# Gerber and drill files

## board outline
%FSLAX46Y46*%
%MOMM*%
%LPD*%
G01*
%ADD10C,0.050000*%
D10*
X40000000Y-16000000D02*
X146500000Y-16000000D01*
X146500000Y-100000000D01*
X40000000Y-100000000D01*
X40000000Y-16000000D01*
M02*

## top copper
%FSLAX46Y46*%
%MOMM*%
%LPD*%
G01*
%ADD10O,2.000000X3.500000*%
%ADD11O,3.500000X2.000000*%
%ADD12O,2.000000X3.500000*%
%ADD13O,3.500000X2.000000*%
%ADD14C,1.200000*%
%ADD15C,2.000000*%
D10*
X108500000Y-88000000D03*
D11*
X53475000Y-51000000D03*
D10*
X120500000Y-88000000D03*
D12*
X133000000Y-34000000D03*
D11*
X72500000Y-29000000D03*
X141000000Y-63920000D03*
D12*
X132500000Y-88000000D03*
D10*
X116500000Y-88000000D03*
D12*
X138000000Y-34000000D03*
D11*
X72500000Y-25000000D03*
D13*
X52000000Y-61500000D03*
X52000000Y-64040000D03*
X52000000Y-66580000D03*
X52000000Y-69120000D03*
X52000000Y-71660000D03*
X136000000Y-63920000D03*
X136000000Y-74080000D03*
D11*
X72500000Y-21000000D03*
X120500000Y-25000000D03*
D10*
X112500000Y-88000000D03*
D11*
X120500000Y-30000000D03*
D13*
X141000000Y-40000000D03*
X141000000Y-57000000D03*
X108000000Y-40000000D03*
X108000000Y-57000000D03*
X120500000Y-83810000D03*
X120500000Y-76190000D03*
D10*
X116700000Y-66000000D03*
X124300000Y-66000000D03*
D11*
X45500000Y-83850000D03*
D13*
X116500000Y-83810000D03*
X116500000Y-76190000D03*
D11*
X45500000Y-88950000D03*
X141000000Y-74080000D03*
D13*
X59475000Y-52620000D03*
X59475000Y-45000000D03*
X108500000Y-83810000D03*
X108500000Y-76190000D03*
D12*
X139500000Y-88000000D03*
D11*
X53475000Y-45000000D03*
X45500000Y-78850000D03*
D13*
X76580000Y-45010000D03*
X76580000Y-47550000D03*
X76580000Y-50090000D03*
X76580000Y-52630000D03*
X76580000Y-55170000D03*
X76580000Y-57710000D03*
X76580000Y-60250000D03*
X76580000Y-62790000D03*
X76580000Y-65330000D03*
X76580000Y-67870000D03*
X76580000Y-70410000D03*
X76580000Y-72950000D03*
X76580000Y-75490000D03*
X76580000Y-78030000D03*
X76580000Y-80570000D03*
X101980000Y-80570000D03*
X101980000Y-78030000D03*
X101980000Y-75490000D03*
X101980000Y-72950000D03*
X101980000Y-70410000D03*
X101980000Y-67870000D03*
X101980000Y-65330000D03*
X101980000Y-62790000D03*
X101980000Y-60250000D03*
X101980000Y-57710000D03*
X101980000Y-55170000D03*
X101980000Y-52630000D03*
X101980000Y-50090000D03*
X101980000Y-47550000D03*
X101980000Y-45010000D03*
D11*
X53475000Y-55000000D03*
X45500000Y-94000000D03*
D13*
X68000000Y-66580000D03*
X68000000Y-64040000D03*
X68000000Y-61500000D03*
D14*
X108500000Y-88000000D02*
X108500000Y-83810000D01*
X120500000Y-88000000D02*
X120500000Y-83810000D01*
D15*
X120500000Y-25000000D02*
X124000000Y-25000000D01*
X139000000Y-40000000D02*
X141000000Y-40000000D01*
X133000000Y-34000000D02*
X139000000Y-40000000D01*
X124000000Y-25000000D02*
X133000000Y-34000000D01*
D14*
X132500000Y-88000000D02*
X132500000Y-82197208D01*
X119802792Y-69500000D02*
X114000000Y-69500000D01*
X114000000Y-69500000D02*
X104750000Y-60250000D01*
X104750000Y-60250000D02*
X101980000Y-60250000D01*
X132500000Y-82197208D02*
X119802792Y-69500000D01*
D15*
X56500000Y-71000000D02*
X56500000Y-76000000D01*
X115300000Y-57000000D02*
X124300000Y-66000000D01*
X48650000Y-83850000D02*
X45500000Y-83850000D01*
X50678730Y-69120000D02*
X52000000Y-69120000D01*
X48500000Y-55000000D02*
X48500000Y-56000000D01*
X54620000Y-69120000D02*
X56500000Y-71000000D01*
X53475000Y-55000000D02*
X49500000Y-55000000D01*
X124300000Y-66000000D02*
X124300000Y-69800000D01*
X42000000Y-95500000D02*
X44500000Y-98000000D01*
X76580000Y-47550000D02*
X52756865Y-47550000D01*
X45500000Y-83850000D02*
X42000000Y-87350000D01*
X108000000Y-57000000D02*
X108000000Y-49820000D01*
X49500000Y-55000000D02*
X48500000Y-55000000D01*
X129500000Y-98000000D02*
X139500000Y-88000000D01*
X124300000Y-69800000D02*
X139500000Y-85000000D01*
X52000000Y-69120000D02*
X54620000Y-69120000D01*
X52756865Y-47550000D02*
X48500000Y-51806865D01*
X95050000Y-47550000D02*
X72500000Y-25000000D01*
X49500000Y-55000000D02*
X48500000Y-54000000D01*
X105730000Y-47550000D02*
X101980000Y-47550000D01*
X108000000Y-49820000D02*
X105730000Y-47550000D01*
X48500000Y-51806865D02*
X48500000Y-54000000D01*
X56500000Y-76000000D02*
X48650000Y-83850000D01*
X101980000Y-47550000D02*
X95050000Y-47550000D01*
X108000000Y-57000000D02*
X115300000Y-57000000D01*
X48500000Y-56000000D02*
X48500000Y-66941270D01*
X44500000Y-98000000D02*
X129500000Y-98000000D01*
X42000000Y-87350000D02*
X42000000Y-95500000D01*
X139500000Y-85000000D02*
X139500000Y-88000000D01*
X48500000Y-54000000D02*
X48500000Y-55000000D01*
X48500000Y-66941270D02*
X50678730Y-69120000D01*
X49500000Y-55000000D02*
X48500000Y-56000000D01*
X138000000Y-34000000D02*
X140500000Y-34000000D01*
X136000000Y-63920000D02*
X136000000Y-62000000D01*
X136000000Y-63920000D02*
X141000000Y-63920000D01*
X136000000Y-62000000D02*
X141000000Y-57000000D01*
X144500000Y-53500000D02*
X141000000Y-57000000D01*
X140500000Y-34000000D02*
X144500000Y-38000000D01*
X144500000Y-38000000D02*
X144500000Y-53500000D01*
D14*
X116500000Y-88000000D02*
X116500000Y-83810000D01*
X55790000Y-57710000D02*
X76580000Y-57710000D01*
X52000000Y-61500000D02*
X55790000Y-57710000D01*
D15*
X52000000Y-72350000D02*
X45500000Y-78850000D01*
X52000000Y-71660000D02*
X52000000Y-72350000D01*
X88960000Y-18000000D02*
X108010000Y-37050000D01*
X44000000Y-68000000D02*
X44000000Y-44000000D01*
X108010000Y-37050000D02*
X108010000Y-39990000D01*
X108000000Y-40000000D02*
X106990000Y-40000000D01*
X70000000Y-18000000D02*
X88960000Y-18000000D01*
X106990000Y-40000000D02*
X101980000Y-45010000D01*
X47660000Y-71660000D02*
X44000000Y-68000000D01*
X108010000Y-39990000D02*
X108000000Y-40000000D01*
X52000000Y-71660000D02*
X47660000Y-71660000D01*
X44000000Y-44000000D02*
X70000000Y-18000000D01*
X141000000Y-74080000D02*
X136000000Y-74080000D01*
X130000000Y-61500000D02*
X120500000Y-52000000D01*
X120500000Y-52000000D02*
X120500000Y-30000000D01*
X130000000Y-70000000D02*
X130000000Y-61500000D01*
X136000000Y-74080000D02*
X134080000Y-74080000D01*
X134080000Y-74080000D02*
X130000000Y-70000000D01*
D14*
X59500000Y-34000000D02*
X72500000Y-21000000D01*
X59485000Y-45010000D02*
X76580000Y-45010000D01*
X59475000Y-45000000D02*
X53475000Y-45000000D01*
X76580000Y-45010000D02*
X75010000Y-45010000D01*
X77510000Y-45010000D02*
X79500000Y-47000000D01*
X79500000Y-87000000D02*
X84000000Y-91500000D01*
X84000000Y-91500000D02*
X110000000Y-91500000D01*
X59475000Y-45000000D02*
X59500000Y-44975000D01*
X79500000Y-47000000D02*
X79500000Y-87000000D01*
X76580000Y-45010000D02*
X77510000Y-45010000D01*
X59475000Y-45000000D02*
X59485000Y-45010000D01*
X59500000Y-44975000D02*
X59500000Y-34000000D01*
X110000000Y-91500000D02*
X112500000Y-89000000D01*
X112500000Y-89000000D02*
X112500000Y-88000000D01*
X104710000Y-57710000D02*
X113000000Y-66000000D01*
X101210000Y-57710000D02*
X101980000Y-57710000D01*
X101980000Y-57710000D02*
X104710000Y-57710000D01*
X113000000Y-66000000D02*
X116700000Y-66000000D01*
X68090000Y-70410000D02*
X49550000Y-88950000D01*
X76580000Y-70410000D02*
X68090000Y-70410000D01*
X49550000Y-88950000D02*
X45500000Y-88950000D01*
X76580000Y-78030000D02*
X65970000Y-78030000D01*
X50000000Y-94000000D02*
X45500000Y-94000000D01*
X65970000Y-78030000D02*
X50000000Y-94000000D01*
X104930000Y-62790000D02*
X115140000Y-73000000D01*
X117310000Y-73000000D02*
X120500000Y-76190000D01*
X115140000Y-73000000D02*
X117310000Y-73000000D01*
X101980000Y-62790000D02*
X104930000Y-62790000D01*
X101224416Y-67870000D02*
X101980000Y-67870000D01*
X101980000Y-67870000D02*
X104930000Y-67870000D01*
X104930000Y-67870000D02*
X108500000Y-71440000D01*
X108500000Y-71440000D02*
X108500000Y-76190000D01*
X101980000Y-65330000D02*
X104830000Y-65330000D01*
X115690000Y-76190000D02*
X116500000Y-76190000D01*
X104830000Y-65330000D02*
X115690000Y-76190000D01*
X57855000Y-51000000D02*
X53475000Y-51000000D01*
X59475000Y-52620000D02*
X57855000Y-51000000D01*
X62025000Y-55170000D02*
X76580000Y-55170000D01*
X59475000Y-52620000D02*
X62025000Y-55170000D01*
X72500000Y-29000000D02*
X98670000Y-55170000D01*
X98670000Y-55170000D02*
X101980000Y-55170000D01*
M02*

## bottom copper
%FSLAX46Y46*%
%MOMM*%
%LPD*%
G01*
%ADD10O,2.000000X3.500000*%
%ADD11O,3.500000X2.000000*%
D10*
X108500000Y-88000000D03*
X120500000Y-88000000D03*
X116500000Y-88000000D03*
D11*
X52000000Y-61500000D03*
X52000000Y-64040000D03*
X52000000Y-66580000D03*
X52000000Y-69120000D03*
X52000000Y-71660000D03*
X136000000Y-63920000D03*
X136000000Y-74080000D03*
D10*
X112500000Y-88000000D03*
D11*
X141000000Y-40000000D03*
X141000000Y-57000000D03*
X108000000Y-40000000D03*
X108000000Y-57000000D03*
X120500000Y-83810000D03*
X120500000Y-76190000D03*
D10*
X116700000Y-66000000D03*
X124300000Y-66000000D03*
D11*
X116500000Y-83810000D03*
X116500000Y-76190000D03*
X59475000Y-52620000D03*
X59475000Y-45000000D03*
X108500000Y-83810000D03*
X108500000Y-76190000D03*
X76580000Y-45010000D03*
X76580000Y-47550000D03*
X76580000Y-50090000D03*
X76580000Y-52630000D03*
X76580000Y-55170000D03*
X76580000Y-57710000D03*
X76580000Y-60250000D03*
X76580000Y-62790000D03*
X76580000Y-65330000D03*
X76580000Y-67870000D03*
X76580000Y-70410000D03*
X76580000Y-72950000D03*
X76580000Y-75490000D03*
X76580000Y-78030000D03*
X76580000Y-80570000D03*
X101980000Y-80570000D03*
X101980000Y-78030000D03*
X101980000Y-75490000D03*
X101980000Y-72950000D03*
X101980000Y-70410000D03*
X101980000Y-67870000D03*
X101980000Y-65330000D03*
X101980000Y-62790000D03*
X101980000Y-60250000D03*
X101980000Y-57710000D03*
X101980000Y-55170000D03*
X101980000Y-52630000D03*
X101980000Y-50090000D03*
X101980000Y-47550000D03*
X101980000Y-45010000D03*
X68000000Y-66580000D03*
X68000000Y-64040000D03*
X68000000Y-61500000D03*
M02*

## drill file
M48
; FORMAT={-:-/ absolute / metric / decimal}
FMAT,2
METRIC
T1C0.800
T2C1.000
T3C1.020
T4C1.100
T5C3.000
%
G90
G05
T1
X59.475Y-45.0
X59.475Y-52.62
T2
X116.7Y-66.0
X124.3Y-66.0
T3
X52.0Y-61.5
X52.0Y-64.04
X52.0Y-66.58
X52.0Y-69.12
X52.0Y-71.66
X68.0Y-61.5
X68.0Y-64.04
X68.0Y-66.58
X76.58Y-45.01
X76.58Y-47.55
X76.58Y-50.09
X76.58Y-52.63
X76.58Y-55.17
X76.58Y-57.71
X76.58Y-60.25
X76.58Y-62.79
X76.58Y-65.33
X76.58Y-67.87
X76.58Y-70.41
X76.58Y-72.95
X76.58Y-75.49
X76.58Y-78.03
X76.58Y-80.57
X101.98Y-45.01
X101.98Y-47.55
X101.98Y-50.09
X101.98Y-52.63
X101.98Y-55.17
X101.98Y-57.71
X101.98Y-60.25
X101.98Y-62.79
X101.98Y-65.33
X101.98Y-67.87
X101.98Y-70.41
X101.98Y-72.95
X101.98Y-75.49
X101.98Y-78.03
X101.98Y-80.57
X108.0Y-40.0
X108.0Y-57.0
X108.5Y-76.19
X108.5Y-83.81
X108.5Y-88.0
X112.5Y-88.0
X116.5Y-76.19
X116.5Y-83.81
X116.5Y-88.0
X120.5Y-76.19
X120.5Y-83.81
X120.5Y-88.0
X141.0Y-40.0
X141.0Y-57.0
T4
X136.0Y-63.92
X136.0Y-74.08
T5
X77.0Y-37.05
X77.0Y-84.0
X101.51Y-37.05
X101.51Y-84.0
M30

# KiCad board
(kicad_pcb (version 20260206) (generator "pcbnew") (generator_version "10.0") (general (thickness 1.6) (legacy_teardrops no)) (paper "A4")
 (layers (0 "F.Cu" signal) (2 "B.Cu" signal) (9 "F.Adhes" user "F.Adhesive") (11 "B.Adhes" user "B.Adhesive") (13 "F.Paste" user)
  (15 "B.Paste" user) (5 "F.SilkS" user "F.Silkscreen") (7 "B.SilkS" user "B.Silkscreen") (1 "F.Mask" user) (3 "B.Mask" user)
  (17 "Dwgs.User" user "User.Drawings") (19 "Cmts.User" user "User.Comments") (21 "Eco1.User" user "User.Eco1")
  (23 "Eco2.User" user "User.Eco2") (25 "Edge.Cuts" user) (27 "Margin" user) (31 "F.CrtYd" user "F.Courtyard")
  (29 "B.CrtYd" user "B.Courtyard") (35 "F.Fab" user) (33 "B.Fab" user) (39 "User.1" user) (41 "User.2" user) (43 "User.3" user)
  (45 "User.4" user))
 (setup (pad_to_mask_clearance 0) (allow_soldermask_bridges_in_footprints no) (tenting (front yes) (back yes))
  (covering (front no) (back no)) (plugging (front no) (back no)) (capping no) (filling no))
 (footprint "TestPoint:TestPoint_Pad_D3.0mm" (layer "F.Cu") (at 108.5 88 -90)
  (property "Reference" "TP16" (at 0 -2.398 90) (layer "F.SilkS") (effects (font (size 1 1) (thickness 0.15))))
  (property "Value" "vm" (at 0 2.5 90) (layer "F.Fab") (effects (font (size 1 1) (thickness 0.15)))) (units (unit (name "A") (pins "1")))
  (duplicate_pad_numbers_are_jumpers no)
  (pad "1" thru_hole oval (at 0 0 270) (size 3.5 2) (drill 1.02) (layers "*.Cu" "*.Mask") (remove_unused_layers no) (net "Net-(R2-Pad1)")
   (solder_mask_margin 0.102) (thermal_bridge_angle 45)))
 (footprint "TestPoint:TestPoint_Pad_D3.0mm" (layer "F.Cu") (at 53.475 51)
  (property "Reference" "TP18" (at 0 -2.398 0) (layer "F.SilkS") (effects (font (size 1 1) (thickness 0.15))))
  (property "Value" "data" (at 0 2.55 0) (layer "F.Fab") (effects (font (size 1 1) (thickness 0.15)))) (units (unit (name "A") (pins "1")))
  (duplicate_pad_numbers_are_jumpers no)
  (pad "1" smd oval (at 0 0) (size 3.5 2) (layers "F.Cu" "F.Mask") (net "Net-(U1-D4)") (thermal_bridge_angle 45)))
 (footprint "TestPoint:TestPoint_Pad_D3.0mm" (layer "F.Cu") (at 120.5 88 -90)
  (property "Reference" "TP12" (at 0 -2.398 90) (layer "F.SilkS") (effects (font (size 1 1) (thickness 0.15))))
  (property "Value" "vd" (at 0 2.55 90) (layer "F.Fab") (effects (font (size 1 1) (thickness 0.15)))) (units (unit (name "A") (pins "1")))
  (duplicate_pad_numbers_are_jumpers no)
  (pad "1" thru_hole oval (at 0 0 270) (size 3.5 2) (drill 1.02) (layers "*.Cu" "*.Mask") (remove_unused_layers no) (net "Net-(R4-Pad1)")
   (solder_mask_margin 0.102) (thermal_bridge_angle 45)))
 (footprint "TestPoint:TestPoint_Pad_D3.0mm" (layer "F.Cu") (at 133 34 90)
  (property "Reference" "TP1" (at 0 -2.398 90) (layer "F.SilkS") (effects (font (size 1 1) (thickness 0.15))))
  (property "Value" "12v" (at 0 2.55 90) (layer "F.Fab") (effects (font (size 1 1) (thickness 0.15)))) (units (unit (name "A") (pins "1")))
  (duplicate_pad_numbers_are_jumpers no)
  (pad "1" smd oval (at 0 0 90) (size 3.5 2) (layers "F.Cu" "F.Mask") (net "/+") (thermal_bridge_angle 45)))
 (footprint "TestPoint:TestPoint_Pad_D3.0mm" (layer "F.Cu") (at 72.5 29 180)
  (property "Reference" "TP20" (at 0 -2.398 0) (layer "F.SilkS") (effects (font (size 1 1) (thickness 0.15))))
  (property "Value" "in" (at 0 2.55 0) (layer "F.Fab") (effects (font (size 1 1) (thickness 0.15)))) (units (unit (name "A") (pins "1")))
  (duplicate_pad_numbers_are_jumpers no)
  (pad "1" smd oval (at 0 0 180) (size 3.5 2) (layers "F.Cu" "F.Mask") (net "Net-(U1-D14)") (thermal_bridge_angle 45)))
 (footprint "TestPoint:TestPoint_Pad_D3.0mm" (layer "F.Cu") (at 141 63.92 180)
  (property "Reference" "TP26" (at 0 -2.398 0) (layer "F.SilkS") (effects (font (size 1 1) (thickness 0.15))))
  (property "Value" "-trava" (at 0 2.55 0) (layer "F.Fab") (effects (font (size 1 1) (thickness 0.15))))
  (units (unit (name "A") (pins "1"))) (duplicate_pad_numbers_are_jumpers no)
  (pad "1" smd oval (at 0 0 180) (size 3.5 2) (layers "F.Cu" "F.Mask") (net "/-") (thermal_bridge_angle 45)))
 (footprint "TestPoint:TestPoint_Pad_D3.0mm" (layer "F.Cu") (at 132.5 88)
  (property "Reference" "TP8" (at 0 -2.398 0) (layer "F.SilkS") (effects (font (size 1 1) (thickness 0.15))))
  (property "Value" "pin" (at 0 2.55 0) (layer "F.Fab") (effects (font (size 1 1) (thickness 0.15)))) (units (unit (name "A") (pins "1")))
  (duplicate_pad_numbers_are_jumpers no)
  (pad "1" smd oval (at 0 0) (size 2 3.5) (layers "F.Cu" "F.Mask") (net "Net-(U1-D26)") (thermal_bridge_angle 45)))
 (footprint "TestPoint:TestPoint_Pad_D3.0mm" (layer "F.Cu") (at 116.5 88 -90)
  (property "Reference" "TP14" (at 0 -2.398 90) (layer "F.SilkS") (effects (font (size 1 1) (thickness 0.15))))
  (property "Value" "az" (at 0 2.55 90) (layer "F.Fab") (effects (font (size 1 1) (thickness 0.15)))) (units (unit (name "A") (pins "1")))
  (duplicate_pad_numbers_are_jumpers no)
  (pad "1" thru_hole oval (at 0 0 270) (size 3.5 2) (drill 1.02) (layers "*.Cu" "*.Mask") (remove_unused_layers no) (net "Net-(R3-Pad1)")
   (solder_mask_margin 0.102) (thermal_bridge_angle 45)))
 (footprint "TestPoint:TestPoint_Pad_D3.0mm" (layer "F.Cu") (at 138 34 90)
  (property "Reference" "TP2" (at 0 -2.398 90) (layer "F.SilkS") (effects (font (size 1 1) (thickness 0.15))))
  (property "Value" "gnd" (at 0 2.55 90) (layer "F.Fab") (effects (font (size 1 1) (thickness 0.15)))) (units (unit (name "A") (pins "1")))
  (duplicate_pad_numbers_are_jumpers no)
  (pad "1" smd oval (at 0 0 90) (size 3.5 2) (layers "F.Cu" "F.Mask") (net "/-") (thermal_bridge_angle 45)))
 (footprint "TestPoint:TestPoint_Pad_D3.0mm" (layer "F.Cu") (at 72.5 25 180)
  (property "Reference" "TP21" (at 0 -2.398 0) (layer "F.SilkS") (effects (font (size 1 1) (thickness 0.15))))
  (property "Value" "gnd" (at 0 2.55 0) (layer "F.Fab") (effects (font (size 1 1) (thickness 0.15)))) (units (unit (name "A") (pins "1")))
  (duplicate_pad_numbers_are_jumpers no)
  (pad "1" smd oval (at 0 0 180) (size 3.5 2) (layers "F.Cu" "F.Mask") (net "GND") (thermal_bridge_angle 45)))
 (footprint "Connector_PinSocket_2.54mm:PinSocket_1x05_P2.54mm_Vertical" (layer "F.Cu") (at 52 61.5)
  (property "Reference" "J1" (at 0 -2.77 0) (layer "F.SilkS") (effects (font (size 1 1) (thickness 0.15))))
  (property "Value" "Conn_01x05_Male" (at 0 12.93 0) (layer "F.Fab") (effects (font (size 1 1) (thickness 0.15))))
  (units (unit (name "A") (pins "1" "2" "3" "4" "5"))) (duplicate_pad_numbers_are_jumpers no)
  (pad "1" thru_hole oval (at 0 0) (size 3.5 2) (drill 1.02) (layers "*.Cu" "*.Mask") (remove_unused_layers no) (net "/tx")
   (solder_mask_margin 0.102) (thermal_bridge_angle 45))
  (pad "2" thru_hole oval (at 0 2.54) (size 3.5 2) (drill 1.02) (layers "*.Cu" "*.Mask") (remove_unused_layers no)
   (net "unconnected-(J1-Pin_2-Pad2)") (solder_mask_margin 0.102) (thermal_bridge_angle 45))
  (pad "3" thru_hole oval (at 0 5.08) (size 3.5 2) (drill 1.02) (layers "*.Cu" "*.Mask") (remove_unused_layers no)
   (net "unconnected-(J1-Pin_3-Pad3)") (solder_mask_margin 0.102) (thermal_bridge_angle 45))
  (pad "4" thru_hole oval (at 0 7.62) (size 3.5 2) (drill 1.02) (layers "*.Cu" "*.Mask") (remove_unused_layers no) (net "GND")
   (solder_mask_margin 0.102) (thermal_bridge_angle 45))
  (pad "5" thru_hole oval (at 0 10.16) (size 3.5 2) (drill 1.02) (layers "*.Cu" "*.Mask") (remove_unused_layers no) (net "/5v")
   (solder_mask_margin 0.102) (thermal_bridge_angle 45)))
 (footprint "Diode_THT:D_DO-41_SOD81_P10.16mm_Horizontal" (layer "F.Cu") (at 136 63.92 -90)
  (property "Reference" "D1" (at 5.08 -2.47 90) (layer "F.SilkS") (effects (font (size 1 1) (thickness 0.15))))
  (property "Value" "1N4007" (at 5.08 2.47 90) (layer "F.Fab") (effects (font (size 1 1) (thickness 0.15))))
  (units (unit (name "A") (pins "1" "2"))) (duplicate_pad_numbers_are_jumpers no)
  (pad "1" thru_hole oval (at 0 0 270) (size 2 3.5) (drill 1.1) (layers "*.Cu" "*.Mask") (remove_unused_layers no) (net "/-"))
  (pad "2" thru_hole oval (at 10.16 0 270) (size 2 3.5) (drill 1.1) (layers "*.Cu" "*.Mask") (remove_unused_layers no) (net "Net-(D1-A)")))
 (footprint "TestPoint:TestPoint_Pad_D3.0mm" (layer "F.Cu") (at 72.5 21 180)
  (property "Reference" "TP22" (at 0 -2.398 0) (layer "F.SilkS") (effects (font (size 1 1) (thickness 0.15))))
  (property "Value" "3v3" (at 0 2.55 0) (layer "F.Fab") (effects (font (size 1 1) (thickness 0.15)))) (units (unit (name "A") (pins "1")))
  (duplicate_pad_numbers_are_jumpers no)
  (pad "1" smd oval (at 0 0 180) (size 3.5 2) (layers "F.Cu" "F.Mask") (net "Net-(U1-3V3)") (thermal_bridge_angle 45)))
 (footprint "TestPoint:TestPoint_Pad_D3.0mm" (layer "F.Cu") (at 120.5 25 180)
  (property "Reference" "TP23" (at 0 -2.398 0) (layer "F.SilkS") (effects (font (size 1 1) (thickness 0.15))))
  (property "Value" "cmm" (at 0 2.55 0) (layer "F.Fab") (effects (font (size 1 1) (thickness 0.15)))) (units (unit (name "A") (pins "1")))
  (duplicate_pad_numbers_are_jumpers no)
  (pad "1" smd oval (at 0 0 180) (size 3.5 2) (layers "F.Cu" "F.Mask") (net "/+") (thermal_bridge_angle 45)))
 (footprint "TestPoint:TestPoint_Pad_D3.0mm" (layer "F.Cu") (at 112.5 88 -90)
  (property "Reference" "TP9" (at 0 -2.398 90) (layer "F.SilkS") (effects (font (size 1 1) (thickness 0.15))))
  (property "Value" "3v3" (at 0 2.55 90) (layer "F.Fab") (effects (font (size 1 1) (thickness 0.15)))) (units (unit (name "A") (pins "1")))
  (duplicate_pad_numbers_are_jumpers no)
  (pad "1" thru_hole oval (at 0 0 270) (size 3.5 2) (drill 1.02) (layers "*.Cu" "*.Mask") (remove_unused_layers no) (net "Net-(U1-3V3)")
   (solder_mask_margin 0.102) (thermal_bridge_angle 45)))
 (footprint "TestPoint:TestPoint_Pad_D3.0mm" (layer "F.Cu") (at 120.5 30 180)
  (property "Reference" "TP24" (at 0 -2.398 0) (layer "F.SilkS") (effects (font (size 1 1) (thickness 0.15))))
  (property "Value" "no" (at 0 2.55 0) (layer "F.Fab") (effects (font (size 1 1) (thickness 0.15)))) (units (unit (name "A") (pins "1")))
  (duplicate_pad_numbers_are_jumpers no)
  (pad "1" smd oval (at 0 0 180) (size 3.5 2) (layers "F.Cu" "F.Mask") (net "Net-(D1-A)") (thermal_bridge_angle 45)))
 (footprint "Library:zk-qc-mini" (layer "F.Cu") (at 124.5 48 180)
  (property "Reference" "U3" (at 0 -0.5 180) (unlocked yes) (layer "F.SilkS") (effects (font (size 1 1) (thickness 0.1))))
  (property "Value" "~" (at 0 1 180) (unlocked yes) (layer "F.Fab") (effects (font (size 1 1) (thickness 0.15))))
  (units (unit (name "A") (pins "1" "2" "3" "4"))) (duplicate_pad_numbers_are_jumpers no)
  (pad "1" thru_hole oval (at -16.5 8 180) (size 3.5 2) (drill 1.02) (layers "*.Cu" "*.Mask") (remove_unused_layers no) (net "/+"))
  (pad "2" thru_hole oval (at -16.5 -9 180) (size 3.5 2) (drill 1.02) (layers "*.Cu" "*.Mask") (remove_unused_layers no) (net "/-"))
  (pad "3" thru_hole oval (at 16.5 8 180) (size 3.5 2) (drill 1.02) (layers "*.Cu" "*.Mask") (remove_unused_layers no) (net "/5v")
   (thermal_bridge_angle 45))
  (pad "4" thru_hole oval (at 16.5 -9 180) (size 3.5 2) (drill 1.02) (layers "*.Cu" "*.Mask") (remove_unused_layers no) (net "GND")
   (thermal_bridge_angle 45)))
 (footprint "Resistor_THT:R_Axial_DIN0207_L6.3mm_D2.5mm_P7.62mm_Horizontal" (layer "F.Cu") (at 120.5 83.81 90)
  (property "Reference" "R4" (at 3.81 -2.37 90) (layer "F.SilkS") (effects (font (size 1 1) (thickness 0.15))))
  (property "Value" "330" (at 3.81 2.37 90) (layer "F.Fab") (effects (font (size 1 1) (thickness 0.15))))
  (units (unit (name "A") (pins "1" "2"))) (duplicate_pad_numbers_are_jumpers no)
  (pad "1" thru_hole oval (at 0 0 90) (size 2 3.5) (drill 1.02) (layers "*.Cu" "*.Mask") (remove_unused_layers no) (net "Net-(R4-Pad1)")
   (solder_mask_margin 0.102) (thermal_bridge_angle 45))
  (pad "2" thru_hole oval (at 7.62 0 90) (size 2 3.5) (drill 1.02) (layers "*.Cu" "*.Mask") (remove_unused_layers no) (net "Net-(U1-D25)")
   (solder_mask_margin 0.102) (thermal_bridge_angle 45)))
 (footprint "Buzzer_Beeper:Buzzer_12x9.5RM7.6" (layer "F.Cu") (at 116.7 66)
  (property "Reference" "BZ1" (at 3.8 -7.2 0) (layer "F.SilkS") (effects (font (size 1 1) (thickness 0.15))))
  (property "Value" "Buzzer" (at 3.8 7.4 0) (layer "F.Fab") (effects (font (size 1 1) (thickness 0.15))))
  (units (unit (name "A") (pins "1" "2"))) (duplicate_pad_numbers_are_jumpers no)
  (pad "1" thru_hole oval (at 0 0) (size 2 3.5) (drill 1) (layers "*.Cu" "*.Mask") (remove_unused_layers no) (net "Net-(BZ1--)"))
  (pad "2" thru_hole oval (at 7.6 0) (size 2 3.5) (drill 1) (layers "*.Cu" "*.Mask") (remove_unused_layers no) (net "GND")
   (thermal_bridge_angle 45)))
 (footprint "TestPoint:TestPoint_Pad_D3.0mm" (layer "F.Cu") (at 45.5 83.85)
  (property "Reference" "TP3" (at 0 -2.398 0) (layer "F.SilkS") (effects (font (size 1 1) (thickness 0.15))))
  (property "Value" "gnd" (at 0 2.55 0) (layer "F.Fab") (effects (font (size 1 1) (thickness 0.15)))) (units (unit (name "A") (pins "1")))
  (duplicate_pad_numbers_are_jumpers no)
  (pad "1" smd oval (at 0 0) (size 3.5 2) (layers "F.Cu" "F.Mask") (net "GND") (thermal_bridge_angle 45)))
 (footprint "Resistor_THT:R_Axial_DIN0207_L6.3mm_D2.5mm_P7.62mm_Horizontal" (layer "F.Cu") (at 116.5 83.81 90)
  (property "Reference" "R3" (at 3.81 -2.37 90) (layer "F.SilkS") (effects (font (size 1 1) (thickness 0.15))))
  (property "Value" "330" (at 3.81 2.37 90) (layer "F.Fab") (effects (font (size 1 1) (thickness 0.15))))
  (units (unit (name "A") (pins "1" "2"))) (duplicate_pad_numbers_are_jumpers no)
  (pad "1" thru_hole oval (at 0 0 90) (size 2 3.5) (drill 1.02) (layers "*.Cu" "*.Mask") (remove_unused_layers no) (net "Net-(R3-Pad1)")
   (solder_mask_margin 0.102) (thermal_bridge_angle 45))
  (pad "2" thru_hole oval (at 7.62 0 90) (size 2 3.5) (drill 1.02) (layers "*.Cu" "*.Mask") (remove_unused_layers no) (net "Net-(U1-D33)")
   (solder_mask_margin 0.102) (thermal_bridge_angle 45)))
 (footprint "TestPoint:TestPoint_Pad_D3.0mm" (layer "F.Cu") (at 45.5 88.95)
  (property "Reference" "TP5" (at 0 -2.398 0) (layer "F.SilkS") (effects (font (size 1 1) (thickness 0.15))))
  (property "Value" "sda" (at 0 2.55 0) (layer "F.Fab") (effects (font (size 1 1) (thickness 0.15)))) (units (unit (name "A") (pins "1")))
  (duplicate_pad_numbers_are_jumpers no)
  (pad "1" smd oval (at 0 0) (size 3.5 2) (layers "F.Cu" "F.Mask") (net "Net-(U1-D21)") (thermal_bridge_angle 45)))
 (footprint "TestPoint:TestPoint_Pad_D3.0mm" (layer "F.Cu") (at 141 74.08 180)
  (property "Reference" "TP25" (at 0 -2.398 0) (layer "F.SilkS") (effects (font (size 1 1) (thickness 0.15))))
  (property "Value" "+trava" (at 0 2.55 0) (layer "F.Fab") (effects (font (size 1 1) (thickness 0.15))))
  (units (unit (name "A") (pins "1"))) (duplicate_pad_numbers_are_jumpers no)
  (pad "1" smd oval (at 0 0 180) (size 3.5 2) (layers "F.Cu" "F.Mask") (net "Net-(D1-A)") (thermal_bridge_angle 45)))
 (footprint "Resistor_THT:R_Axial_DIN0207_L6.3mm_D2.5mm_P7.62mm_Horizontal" (layer "F.Cu") (at 59.475 52.62 90)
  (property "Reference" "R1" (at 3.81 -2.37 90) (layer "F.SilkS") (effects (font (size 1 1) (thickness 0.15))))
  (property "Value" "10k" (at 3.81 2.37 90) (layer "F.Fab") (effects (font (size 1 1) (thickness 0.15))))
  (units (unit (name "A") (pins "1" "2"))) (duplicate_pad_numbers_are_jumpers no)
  (pad "1" thru_hole oval (at 0 0 90) (size 2 3.5) (drill 0.8) (layers "*.Cu" "*.Mask") (remove_unused_layers no) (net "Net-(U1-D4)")
   (thermal_bridge_angle 45))
  (pad "2" thru_hole oval (at 7.62 0 90) (size 2 3.5) (drill 0.8) (layers "*.Cu" "*.Mask") (remove_unused_layers no) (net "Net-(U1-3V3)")))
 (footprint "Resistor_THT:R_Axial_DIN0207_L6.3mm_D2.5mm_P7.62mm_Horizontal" (layer "F.Cu") (at 108.5 83.81 90)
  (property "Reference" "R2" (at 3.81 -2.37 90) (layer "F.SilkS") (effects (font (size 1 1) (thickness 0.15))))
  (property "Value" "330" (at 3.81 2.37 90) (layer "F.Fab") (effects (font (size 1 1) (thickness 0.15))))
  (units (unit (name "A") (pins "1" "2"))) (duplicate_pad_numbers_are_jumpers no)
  (pad "1" thru_hole oval (at 0 0 90) (size 2 3.5) (drill 1.02) (layers "*.Cu" "*.Mask") (remove_unused_layers no) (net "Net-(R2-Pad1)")
   (solder_mask_margin 0.102) (thermal_bridge_angle 45))
  (pad "2" thru_hole oval (at 7.62 0 90) (size 2 3.5) (drill 1.02) (layers "*.Cu" "*.Mask") (remove_unused_layers no) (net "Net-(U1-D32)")
   (solder_mask_margin 0.102) (thermal_bridge_angle 45)))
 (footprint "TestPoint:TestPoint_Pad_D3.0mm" (layer "F.Cu") (at 139.5 88)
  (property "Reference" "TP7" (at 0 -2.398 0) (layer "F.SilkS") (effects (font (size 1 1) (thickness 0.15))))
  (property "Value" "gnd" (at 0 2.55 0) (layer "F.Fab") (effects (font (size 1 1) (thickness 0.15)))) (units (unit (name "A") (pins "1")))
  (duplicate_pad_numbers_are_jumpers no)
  (pad "1" smd oval (at 0 0) (size 2 3.5) (layers "F.Cu" "F.Mask") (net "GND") (thermal_bridge_angle 45)))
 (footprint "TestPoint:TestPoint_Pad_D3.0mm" (layer "F.Cu") (at 53.475 45)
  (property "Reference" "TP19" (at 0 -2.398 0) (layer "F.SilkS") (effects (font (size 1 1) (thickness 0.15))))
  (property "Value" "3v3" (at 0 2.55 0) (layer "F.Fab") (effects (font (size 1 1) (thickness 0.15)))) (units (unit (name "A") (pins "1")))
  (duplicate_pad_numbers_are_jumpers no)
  (pad "1" smd oval (at 0 0) (size 3.5 2) (layers "F.Cu" "F.Mask") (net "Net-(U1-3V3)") (thermal_bridge_angle 45)))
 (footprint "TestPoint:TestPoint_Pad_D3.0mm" (layer "F.Cu") (at 45.5 78.85)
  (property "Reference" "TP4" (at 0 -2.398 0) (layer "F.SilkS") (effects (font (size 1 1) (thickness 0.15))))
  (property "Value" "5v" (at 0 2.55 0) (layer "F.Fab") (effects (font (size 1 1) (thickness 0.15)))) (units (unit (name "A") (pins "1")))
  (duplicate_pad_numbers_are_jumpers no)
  (pad "1" smd oval (at 0 0) (size 3.5 2) (layers "F.Cu" "F.Mask") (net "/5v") (thermal_bridge_angle 45)))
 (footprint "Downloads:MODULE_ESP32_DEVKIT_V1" (layer "F.Cu") (at 89.28 60.525)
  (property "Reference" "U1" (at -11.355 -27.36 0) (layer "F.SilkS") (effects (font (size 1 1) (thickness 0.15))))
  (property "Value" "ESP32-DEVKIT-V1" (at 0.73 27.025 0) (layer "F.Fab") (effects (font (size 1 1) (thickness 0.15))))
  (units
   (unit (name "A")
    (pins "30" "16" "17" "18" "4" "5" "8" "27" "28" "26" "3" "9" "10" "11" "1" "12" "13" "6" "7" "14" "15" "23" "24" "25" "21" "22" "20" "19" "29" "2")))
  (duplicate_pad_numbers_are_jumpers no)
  (pad "" np_thru_hole circle (at -12.28 -23.475) (size 3 3) (drill 3) (layers "*.Cu" "*.Mask"))
  (pad "" np_thru_hole circle (at -12.28 23.475) (size 3 3) (drill 3) (layers "*.Cu" "*.Mask"))
  (pad "" np_thru_hole circle (at 12.23 -23.475) (size 3 3) (drill 3) (layers "*.Cu" "*.Mask"))
  (pad "" np_thru_hole circle (at 12.23 23.475) (size 3 3) (drill 3) (layers "*.Cu" "*.Mask"))
  (pad "1" thru_hole oval (at -12.7 -15.515) (size 3.5 2) (drill 1.02) (layers "*.Cu" "*.Mask") (remove_unused_layers no)
   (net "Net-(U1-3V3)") (solder_mask_margin 0.102) (thermal_bridge_angle 45))
  (pad "2" thru_hole oval (at -12.7 -12.975) (size 3.5 2) (drill 1.02) (layers "*.Cu" "*.Mask") (remove_unused_layers no) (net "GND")
   (solder_mask_margin 0.102) (thermal_bridge_angle 45))
  (pad "3" thru_hole oval (at -12.7 -10.435) (size 3.5 2) (drill 1.02) (layers "*.Cu" "*.Mask") (remove_unused_layers no)
   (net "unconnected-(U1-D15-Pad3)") (solder_mask_margin 0.102) (thermal_bridge_angle 45))
  (pad "4" thru_hole oval (at -12.7 -7.895) (size 3.5 2) (drill 1.02) (layers "*.Cu" "*.Mask") (remove_unused_layers no)
   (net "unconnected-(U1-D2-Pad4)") (solder_mask_margin 0.102) (thermal_bridge_angle 45))
  (pad "5" thru_hole oval (at -12.7 -5.355) (size 3.5 2) (drill 1.02) (layers "*.Cu" "*.Mask") (remove_unused_layers no) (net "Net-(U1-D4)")
   (solder_mask_margin 0.102) (thermal_bridge_angle 45))
  (pad "6" thru_hole oval (at -12.7 -2.815) (size 3.5 2) (drill 1.02) (layers "*.Cu" "*.Mask") (remove_unused_layers no) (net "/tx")
   (solder_mask_margin 0.102) (thermal_bridge_angle 45))
  (pad "7" thru_hole oval (at -12.7 -0.275) (size 3.5 2) (drill 1.02) (layers "*.Cu" "*.Mask") (remove_unused_layers no)
   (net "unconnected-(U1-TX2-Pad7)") (solder_mask_margin 0.102) (thermal_bridge_angle 45))
  (pad "8" thru_hole oval (at -12.7 2.265) (size 3.5 2) (drill 1.02) (layers "*.Cu" "*.Mask") (remove_unused_layers no)
   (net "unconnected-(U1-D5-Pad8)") (solder_mask_margin 0.102) (thermal_bridge_angle 45))
  (pad "9" thru_hole oval (at -12.7 4.805) (size 3.5 2) (drill 1.02) (layers "*.Cu" "*.Mask") (remove_unused_layers no)
   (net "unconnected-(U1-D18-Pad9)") (solder_mask_margin 0.102) (thermal_bridge_angle 45))
  (pad "10" thru_hole oval (at -12.7 7.345) (size 3.5 2) (drill 1.02) (layers "*.Cu" "*.Mask") (remove_unused_layers no)
   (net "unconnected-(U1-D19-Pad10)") (solder_mask_margin 0.102) (thermal_bridge_angle 45))
  (pad "11" thru_hole oval (at -12.7 9.885) (size 3.5 2) (drill 1.02) (layers "*.Cu" "*.Mask") (remove_unused_layers no)
   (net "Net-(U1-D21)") (solder_mask_margin 0.102) (thermal_bridge_angle 45))
  (pad "12" thru_hole oval (at -12.7 12.425) (size 3.5 2) (drill 1.02) (layers "*.Cu" "*.Mask") (remove_unused_layers no)
   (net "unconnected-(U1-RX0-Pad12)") (solder_mask_margin 0.102) (thermal_bridge_angle 45))
  (pad "13" thru_hole oval (at -12.7 14.965) (size 3.5 2) (drill 1.02) (layers "*.Cu" "*.Mask") (remove_unused_layers no)
   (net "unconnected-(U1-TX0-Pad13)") (solder_mask_margin 0.102) (thermal_bridge_angle 45))
  (pad "14" thru_hole oval (at -12.7 17.505) (size 3.5 2) (drill 1.02) (layers "*.Cu" "*.Mask") (remove_unused_layers no)
   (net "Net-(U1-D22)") (solder_mask_margin 0.102) (thermal_bridge_angle 45))
  (pad "15" thru_hole oval (at -12.7 20.045) (size 3.5 2) (drill 1.02) (layers "*.Cu" "*.Mask") (remove_unused_layers no)
   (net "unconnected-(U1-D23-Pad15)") (solder_mask_margin 0.102) (thermal_bridge_angle 45))
  (pad "16" thru_hole oval (at 12.7 20.045) (size 3.5 2) (drill 1.02) (layers "*.Cu" "*.Mask") (remove_unused_layers no)
   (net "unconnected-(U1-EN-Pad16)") (solder_mask_margin 0.102) (thermal_bridge_angle 45))
  (pad "17" thru_hole oval (at 12.7 17.505) (size 3.5 2) (drill 1.02) (layers "*.Cu" "*.Mask") (remove_unused_layers no)
   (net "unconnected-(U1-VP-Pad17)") (solder_mask_margin 0.102) (thermal_bridge_angle 45))
  (pad "18" thru_hole oval (at 12.7 14.965) (size 3.5 2) (drill 1.02) (layers "*.Cu" "*.Mask") (remove_unused_layers no)
   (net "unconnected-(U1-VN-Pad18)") (solder_mask_margin 0.102) (thermal_bridge_angle 45))
  (pad "19" thru_hole oval (at 12.7 12.425) (size 3.5 2) (drill 1.02) (layers "*.Cu" "*.Mask") (remove_unused_layers no)
   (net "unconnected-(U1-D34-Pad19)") (solder_mask_margin 0.102) (thermal_bridge_angle 45))
  (pad "20" thru_hole oval (at 12.7 9.885) (size 3.5 2) (drill 1.02) (layers "*.Cu" "*.Mask") (remove_unused_layers no)
   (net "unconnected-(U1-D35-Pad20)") (solder_mask_margin 0.102) (thermal_bridge_angle 45))
  (pad "21" thru_hole oval (at 12.7 7.345) (size 3.5 2) (drill 1.02) (layers "*.Cu" "*.Mask") (remove_unused_layers no) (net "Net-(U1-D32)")
   (solder_mask_margin 0.102) (thermal_bridge_angle 45))
  (pad "22" thru_hole oval (at 12.7 4.805) (size 3.5 2) (drill 1.02) (layers "*.Cu" "*.Mask") (remove_unused_layers no) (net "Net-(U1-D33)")
   (solder_mask_margin 0.102) (thermal_bridge_angle 45))
  (pad "23" thru_hole oval (at 12.7 2.265) (size 3.5 2) (drill 1.02) (layers "*.Cu" "*.Mask") (remove_unused_layers no) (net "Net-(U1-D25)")
   (solder_mask_margin 0.102) (thermal_bridge_angle 45))
  (pad "24" thru_hole oval (at 12.7 -0.275) (size 3.5 2) (drill 1.02) (layers "*.Cu" "*.Mask") (remove_unused_layers no)
   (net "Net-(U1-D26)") (solder_mask_margin 0.102) (thermal_bridge_angle 45))
  (pad "25" thru_hole oval (at 12.7 -2.815) (size 3.5 2) (drill 1.02) (layers "*.Cu" "*.Mask") (remove_unused_layers no) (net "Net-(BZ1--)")
   (solder_mask_margin 0.102) (thermal_bridge_angle 45))
  (pad "26" thru_hole oval (at 12.7 -5.355) (size 3.5 2) (drill 1.02) (layers "*.Cu" "*.Mask") (remove_unused_layers no)
   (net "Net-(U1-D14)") (solder_mask_margin 0.102) (thermal_bridge_angle 45))
  (pad "27" thru_hole oval (at 12.7 -7.895) (size 3.5 2) (drill 1.02) (layers "*.Cu" "*.Mask") (remove_unused_layers no)
   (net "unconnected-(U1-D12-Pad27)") (solder_mask_margin 0.102) (thermal_bridge_angle 45))
  (pad "28" thru_hole oval (at 12.7 -10.435) (size 3.5 2) (drill 1.02) (layers "*.Cu" "*.Mask") (remove_unused_layers no)
   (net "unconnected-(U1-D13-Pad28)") (solder_mask_margin 0.102) (thermal_bridge_angle 45))
  (pad "29" thru_hole oval (at 12.7 -12.975) (size 3.5 2) (drill 1.02) (layers "*.Cu" "*.Mask") (remove_unused_layers no) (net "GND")
   (solder_mask_margin 0.102) (thermal_bridge_angle 45))
  (pad "30" thru_hole oval (at 12.7 -15.515) (size 3.5 2) (drill 1.02) (layers "*.Cu" "*.Mask") (remove_unused_layers no) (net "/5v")
   (solder_mask_margin 0.102) (thermal_bridge_angle 45))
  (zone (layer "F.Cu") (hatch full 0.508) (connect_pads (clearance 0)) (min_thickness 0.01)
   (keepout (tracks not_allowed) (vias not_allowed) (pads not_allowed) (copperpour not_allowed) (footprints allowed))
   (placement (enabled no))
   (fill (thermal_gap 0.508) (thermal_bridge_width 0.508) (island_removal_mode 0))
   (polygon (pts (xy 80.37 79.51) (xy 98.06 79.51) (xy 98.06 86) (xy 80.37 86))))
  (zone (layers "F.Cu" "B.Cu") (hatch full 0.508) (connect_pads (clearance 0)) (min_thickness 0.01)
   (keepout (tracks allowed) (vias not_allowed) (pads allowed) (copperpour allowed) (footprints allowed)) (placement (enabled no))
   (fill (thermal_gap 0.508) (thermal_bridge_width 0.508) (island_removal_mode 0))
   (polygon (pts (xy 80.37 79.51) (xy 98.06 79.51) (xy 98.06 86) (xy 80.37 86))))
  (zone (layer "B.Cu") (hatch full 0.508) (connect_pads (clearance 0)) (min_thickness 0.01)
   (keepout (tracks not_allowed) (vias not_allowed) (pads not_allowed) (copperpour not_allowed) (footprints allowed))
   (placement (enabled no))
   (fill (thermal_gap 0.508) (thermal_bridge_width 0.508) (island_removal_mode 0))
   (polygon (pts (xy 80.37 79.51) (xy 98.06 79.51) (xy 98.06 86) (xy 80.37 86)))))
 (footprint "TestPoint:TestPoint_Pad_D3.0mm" (layer "F.Cu") (at 53.475 55)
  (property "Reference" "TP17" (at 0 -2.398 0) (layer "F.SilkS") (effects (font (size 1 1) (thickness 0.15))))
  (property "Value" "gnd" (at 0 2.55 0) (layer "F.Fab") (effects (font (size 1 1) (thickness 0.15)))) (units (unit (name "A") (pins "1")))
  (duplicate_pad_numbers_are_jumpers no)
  (pad "1" smd oval (at 0 0) (size 3.5 2) (layers "F.Cu" "F.Mask") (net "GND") (thermal_bridge_angle 45)))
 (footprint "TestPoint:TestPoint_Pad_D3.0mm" (layer "F.Cu") (at 45.5 94)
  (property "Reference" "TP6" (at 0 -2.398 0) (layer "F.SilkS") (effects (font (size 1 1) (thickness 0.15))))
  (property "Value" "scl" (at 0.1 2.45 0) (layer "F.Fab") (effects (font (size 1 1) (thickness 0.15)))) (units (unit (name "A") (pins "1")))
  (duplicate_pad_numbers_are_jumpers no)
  (pad "1" smd oval (at 0 0) (size 3.5 2) (layers "F.Cu" "F.Mask") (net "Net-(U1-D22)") (thermal_bridge_angle 45)))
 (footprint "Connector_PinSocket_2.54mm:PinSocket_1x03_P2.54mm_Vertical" (layer "F.Cu") (at 68 66.58 180)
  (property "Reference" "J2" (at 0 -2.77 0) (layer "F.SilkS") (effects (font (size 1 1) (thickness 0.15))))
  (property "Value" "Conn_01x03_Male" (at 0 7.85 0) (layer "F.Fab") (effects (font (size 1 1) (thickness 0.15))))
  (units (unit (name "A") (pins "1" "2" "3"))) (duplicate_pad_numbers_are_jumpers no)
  (pad "1" thru_hole oval (at 0 0 180) (size 3.5 2) (drill 1.02) (layers "*.Cu" "*.Mask") (remove_unused_layers no)
   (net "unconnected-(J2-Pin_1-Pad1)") (solder_mask_margin 0.102) (thermal_bridge_angle 45))
  (pad "2" thru_hole oval (at 0 2.54 180) (size 3.5 2) (drill 1.02) (layers "*.Cu" "*.Mask") (remove_unused_layers no)
   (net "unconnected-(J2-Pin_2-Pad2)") (solder_mask_margin 0.102) (thermal_bridge_angle 45))
  (pad "3" thru_hole oval (at 0 5.08 180) (size 3.5 2) (drill 1.02) (layers "*.Cu" "*.Mask") (remove_unused_layers no)
   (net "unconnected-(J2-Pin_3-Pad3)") (solder_mask_margin 0.102) (thermal_bridge_angle 45)))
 (gr_rect (start 40 16) (end 146.5 100) (stroke (width 0.05) (type default)) (fill no) (layer "Edge.Cuts"))
 (segment (start 108.5 88) (end 108.5 83.81) (width 1.2) (layer "F.Cu") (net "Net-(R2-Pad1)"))
 (segment (start 120.5 88) (end 120.5 83.81) (width 1.2) (layer "F.Cu") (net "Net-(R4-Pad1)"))
 (segment (start 120.5 25) (end 124 25) (width 2) (layer "F.Cu") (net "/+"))
 (segment (start 139 40) (end 141 40) (width 2) (layer "F.Cu") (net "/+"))
 (segment (start 133 34) (end 139 40) (width 2) (layer "F.Cu") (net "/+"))
 (segment (start 124 25) (end 133 34) (width 2) (layer "F.Cu") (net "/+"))
 (segment (start 132.5 88) (end 132.5 82.197208) (width 1.2) (layer "F.Cu") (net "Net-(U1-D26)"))
 (segment (start 119.802792 69.5) (end 114 69.5) (width 1.2) (layer "F.Cu") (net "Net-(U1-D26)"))
 (segment (start 114 69.5) (end 104.75 60.25) (width 1.2) (layer "F.Cu") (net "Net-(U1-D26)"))
 (segment (start 104.75 60.25) (end 101.98 60.25) (width 1.2) (layer "F.Cu") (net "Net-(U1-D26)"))
 (segment (start 132.5 82.197208) (end 119.802792 69.5) (width 1.2) (layer "F.Cu") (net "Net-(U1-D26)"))
 (segment (start 56.5 71) (end 56.5 76) (width 2) (layer "F.Cu") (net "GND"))
 (segment (start 115.3 57) (end 124.3 66) (width 2) (layer "F.Cu") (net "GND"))
 (segment (start 48.65 83.85) (end 45.5 83.85) (width 2) (layer "F.Cu") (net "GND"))
 (segment (start 50.67873 69.12) (end 52 69.12) (width 2) (layer "F.Cu") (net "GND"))
 (segment (start 48.5 55) (end 48.5 56) (width 2) (layer "F.Cu") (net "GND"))
 (segment (start 54.62 69.12) (end 56.5 71) (width 2) (layer "F.Cu") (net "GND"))
 (segment (start 53.475 55) (end 49.5 55) (width 2) (layer "F.Cu") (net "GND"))
 (segment (start 124.3 66) (end 124.3 69.8) (width 2) (layer "F.Cu") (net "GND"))
 (segment (start 42 95.5) (end 44.5 98) (width 2) (layer "F.Cu") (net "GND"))
 (segment (start 76.58 47.55) (end 52.756865 47.55) (width 2) (layer "F.Cu") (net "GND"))
 (segment (start 45.5 83.85) (end 42 87.35) (width 2) (layer "F.Cu") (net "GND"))
 (segment (start 108 57) (end 108 49.82) (width 2) (layer "F.Cu") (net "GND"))
 (segment (start 49.5 55) (end 48.5 55) (width 2) (layer "F.Cu") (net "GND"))
 (segment (start 129.5 98) (end 139.5 88) (width 2) (layer "F.Cu") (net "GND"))
 (segment (start 124.3 69.8) (end 139.5 85) (width 2) (layer "F.Cu") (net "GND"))
 (segment (start 52 69.12) (end 54.62 69.12) (width 2) (layer "F.Cu") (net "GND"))
 (segment (start 52.756865 47.55) (end 48.5 51.806865) (width 2) (layer "F.Cu") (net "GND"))
 (segment (start 95.05 47.55) (end 72.5 25) (width 2) (layer "F.Cu") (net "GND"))
 (segment (start 49.5 55) (end 48.5 54) (width 2) (layer "F.Cu") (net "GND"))
 (segment (start 105.73 47.55) (end 101.98 47.55) (width 2) (layer "F.Cu") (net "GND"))
 (segment (start 108 49.82) (end 105.73 47.55) (width 2) (layer "F.Cu") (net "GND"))
 (segment (start 48.5 51.806865) (end 48.5 54) (width 2) (layer "F.Cu") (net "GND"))
 (segment (start 56.5 76) (end 48.65 83.85) (width 2) (layer "F.Cu") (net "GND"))
 (segment (start 101.98 47.55) (end 95.05 47.55) (width 2) (layer "F.Cu") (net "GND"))
 (segment (start 108 57) (end 115.3 57) (width 2) (layer "F.Cu") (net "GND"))
 (segment (start 48.5 56) (end 48.5 66.94127) (width 2) (layer "F.Cu") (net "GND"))
 (segment (start 44.5 98) (end 129.5 98) (width 2) (layer "F.Cu") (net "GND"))
 (segment (start 42 87.35) (end 42 95.5) (width 2) (layer "F.Cu") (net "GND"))
 (segment (start 139.5 85) (end 139.5 88) (width 2) (layer "F.Cu") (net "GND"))
 (segment (start 48.5 54) (end 48.5 55) (width 2) (layer "F.Cu") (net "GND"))
 (segment (start 48.5 66.94127) (end 50.67873 69.12) (width 2) (layer "F.Cu") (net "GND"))
 (segment (start 49.5 55) (end 48.5 56) (width 2) (layer "F.Cu") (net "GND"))
 (segment (start 138 34) (end 140.5 34) (width 2) (layer "F.Cu") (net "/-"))
 (segment (start 136 63.92) (end 136 62) (width 2) (layer "F.Cu") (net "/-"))
 (segment (start 136 63.92) (end 141 63.92) (width 2) (layer "F.Cu") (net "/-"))
 (segment (start 136 62) (end 141 57) (width 2) (layer "F.Cu") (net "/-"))
 (segment (start 144.5 53.5) (end 141 57) (width 2) (layer "F.Cu") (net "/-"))
 (segment (start 140.5 34) (end 144.5 38) (width 2) (layer "F.Cu") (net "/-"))
 (segment (start 144.5 38) (end 144.5 53.5) (width 2) (layer "F.Cu") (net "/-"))
 (segment (start 116.5 88) (end 116.5 83.81) (width 1.2) (layer "F.Cu") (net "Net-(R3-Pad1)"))
 (segment (start 55.79 57.71) (end 76.58 57.71) (width 1.2) (layer "F.Cu") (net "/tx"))
 (segment (start 52 61.5) (end 55.79 57.71) (width 1.2) (layer "F.Cu") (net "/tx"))
 (segment (start 52 72.35) (end 45.5 78.85) (width 2) (layer "F.Cu") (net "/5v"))
 (segment (start 52 71.66) (end 52 72.35) (width 2) (layer "F.Cu") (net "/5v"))
 (segment (start 88.96 18) (end 108.01 37.05) (width 2) (layer "F.Cu") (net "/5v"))
 (segment (start 44 68) (end 44 44) (width 2) (layer "F.Cu") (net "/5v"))
 (segment (start 108.01 37.05) (end 108.01 39.99) (width 2) (layer "F.Cu") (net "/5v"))
 (segment (start 108 40) (end 106.99 40) (width 2) (layer "F.Cu") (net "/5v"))
 (segment (start 70 18) (end 88.96 18) (width 2) (layer "F.Cu") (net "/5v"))
 (segment (start 106.99 40) (end 101.98 45.01) (width 2) (layer "F.Cu") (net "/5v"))
 (segment (start 47.66 71.66) (end 44 68) (width 2) (layer "F.Cu") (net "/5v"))
 (segment (start 108.01 39.99) (end 108 40) (width 2) (layer "F.Cu") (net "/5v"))
 (segment (start 52 71.66) (end 47.66 71.66) (width 2) (layer "F.Cu") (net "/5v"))
 (segment (start 44 44) (end 70 18) (width 2) (layer "F.Cu") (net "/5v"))
 (segment (start 141 74.08) (end 136 74.08) (width 2) (layer "F.Cu") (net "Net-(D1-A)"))
 (segment (start 130 61.5) (end 120.5 52) (width 2) (layer "F.Cu") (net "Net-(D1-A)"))
 (segment (start 120.5 52) (end 120.5 30) (width 2) (layer "F.Cu") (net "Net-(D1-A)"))
 (segment (start 130 70) (end 130 61.5) (width 2) (layer "F.Cu") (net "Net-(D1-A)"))
 (segment (start 136 74.08) (end 134.08 74.08) (width 2) (layer "F.Cu") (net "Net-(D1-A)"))
 (segment (start 134.08 74.08) (end 130 70) (width 2) (layer "F.Cu") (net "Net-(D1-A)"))
 (segment (start 59.5 34) (end 72.5 21) (width 1.2) (layer "F.Cu") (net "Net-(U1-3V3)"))
 (segment (start 59.485 45.01) (end 76.58 45.01) (width 1.2) (layer "F.Cu") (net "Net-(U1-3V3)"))
 (segment (start 59.475 45) (end 53.475 45) (width 1.2) (layer "F.Cu") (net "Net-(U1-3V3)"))
 (segment (start 76.58 45.01) (end 75.01 45.01) (width 1.2) (layer "F.Cu") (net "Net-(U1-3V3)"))
 (segment (start 77.51 45.01) (end 79.5 47) (width 1.2) (layer "F.Cu") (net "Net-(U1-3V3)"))
 (segment (start 79.5 87) (end 84 91.5) (width 1.2) (layer "F.Cu") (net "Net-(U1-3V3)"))
 (segment (start 84 91.5) (end 110 91.5) (width 1.2) (layer "F.Cu") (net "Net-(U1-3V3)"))
 (segment (start 59.475 45) (end 59.5 44.975) (width 1.2) (layer "F.Cu") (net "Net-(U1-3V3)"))
 (segment (start 79.5 47) (end 79.5 87) (width 1.2) (layer "F.Cu") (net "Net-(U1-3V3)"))
 (segment (start 76.58 45.01) (end 77.51 45.01) (width 1.2) (layer "F.Cu") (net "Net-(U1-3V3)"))
 (segment (start 59.475 45) (end 59.485 45.01) (width 1.2) (layer "F.Cu") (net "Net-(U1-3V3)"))
 (segment (start 59.5 44.975) (end 59.5 34) (width 1.2) (layer "F.Cu") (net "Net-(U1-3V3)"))
 (segment (start 110 91.5) (end 112.5 89) (width 1.2) (layer "F.Cu") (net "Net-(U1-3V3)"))
 (segment (start 112.5 89) (end 112.5 88) (width 1.2) (layer "F.Cu") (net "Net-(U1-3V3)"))
 (segment (start 104.71 57.71) (end 113 66) (width 1.2) (layer "F.Cu") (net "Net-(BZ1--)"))
 (segment (start 101.21 57.71) (end 101.98 57.71) (width 1.2) (layer "F.Cu") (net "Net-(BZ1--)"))
 (segment (start 101.98 57.71) (end 104.71 57.71) (width 1.2) (layer "F.Cu") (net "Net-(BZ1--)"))
 (segment (start 113 66) (end 116.7 66) (width 1.2) (layer "F.Cu") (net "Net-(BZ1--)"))
 (segment (start 68.09 70.41) (end 49.55 88.95) (width 1.2) (layer "F.Cu") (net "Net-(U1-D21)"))
 (segment (start 76.58 70.41) (end 68.09 70.41) (width 1.2) (layer "F.Cu") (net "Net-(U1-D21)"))
 (segment (start 49.55 88.95) (end 45.5 88.95) (width 1.2) (layer "F.Cu") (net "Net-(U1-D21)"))
 (segment (start 76.58 78.03) (end 65.97 78.03) (width 1.2) (layer "F.Cu") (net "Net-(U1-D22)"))
 (segment (start 50 94) (end 45.5 94) (width 1.2) (layer "F.Cu") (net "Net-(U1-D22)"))
 (segment (start 65.97 78.03) (end 50 94) (width 1.2) (layer "F.Cu") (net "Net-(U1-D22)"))
 (segment (start 104.93 62.79) (end 115.14 73) (width 1.2) (layer "F.Cu") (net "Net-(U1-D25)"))
 (segment (start 117.31 73) (end 120.5 76.19) (width 1.2) (layer "F.Cu") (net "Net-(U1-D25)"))
 (segment (start 115.14 73) (end 117.31 73) (width 1.2) (layer "F.Cu") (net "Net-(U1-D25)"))
 (segment (start 101.98 62.79) (end 104.93 62.79) (width 1.2) (layer "F.Cu") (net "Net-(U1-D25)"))
 (segment (start 101.224416 67.87) (end 101.98 67.87) (width 1.2) (layer "F.Cu") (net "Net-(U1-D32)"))
 (segment (start 101.98 67.87) (end 104.93 67.87) (width 1.2) (layer "F.Cu") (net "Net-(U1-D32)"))
 (segment (start 104.93 67.87) (end 108.5 71.44) (width 1.2) (layer "F.Cu") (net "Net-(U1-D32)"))
 (segment (start 108.5 71.44) (end 108.5 76.19) (width 1.2) (layer "F.Cu") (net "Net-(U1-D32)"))
 (segment (start 101.98 65.33) (end 104.83 65.33) (width 1.2) (layer "F.Cu") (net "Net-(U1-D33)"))
 (segment (start 115.69 76.19) (end 116.5 76.19) (width 1.2) (layer "F.Cu") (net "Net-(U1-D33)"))
 (segment (start 104.83 65.33) (end 115.69 76.19) (width 1.2) (layer "F.Cu") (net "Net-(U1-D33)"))
 (segment (start 57.855 51) (end 53.475 51) (width 1.2) (layer "F.Cu") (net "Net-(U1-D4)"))
 (segment (start 59.475 52.62) (end 57.855 51) (width 1.2) (layer "F.Cu") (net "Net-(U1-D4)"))
 (segment (start 62.025 55.17) (end 76.58 55.17) (width 1.2) (layer "F.Cu") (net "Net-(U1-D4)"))
 (segment (start 59.475 52.62) (end 62.025 55.17) (width 1.2) (layer "F.Cu") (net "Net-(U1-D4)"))
 (segment (start 72.5 29) (end 98.67 55.17) (width 1.2) (layer "F.Cu") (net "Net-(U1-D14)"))
 (segment (start 98.67 55.17) (end 101.98 55.17) (width 1.2) (layer "F.Cu") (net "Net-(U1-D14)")))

